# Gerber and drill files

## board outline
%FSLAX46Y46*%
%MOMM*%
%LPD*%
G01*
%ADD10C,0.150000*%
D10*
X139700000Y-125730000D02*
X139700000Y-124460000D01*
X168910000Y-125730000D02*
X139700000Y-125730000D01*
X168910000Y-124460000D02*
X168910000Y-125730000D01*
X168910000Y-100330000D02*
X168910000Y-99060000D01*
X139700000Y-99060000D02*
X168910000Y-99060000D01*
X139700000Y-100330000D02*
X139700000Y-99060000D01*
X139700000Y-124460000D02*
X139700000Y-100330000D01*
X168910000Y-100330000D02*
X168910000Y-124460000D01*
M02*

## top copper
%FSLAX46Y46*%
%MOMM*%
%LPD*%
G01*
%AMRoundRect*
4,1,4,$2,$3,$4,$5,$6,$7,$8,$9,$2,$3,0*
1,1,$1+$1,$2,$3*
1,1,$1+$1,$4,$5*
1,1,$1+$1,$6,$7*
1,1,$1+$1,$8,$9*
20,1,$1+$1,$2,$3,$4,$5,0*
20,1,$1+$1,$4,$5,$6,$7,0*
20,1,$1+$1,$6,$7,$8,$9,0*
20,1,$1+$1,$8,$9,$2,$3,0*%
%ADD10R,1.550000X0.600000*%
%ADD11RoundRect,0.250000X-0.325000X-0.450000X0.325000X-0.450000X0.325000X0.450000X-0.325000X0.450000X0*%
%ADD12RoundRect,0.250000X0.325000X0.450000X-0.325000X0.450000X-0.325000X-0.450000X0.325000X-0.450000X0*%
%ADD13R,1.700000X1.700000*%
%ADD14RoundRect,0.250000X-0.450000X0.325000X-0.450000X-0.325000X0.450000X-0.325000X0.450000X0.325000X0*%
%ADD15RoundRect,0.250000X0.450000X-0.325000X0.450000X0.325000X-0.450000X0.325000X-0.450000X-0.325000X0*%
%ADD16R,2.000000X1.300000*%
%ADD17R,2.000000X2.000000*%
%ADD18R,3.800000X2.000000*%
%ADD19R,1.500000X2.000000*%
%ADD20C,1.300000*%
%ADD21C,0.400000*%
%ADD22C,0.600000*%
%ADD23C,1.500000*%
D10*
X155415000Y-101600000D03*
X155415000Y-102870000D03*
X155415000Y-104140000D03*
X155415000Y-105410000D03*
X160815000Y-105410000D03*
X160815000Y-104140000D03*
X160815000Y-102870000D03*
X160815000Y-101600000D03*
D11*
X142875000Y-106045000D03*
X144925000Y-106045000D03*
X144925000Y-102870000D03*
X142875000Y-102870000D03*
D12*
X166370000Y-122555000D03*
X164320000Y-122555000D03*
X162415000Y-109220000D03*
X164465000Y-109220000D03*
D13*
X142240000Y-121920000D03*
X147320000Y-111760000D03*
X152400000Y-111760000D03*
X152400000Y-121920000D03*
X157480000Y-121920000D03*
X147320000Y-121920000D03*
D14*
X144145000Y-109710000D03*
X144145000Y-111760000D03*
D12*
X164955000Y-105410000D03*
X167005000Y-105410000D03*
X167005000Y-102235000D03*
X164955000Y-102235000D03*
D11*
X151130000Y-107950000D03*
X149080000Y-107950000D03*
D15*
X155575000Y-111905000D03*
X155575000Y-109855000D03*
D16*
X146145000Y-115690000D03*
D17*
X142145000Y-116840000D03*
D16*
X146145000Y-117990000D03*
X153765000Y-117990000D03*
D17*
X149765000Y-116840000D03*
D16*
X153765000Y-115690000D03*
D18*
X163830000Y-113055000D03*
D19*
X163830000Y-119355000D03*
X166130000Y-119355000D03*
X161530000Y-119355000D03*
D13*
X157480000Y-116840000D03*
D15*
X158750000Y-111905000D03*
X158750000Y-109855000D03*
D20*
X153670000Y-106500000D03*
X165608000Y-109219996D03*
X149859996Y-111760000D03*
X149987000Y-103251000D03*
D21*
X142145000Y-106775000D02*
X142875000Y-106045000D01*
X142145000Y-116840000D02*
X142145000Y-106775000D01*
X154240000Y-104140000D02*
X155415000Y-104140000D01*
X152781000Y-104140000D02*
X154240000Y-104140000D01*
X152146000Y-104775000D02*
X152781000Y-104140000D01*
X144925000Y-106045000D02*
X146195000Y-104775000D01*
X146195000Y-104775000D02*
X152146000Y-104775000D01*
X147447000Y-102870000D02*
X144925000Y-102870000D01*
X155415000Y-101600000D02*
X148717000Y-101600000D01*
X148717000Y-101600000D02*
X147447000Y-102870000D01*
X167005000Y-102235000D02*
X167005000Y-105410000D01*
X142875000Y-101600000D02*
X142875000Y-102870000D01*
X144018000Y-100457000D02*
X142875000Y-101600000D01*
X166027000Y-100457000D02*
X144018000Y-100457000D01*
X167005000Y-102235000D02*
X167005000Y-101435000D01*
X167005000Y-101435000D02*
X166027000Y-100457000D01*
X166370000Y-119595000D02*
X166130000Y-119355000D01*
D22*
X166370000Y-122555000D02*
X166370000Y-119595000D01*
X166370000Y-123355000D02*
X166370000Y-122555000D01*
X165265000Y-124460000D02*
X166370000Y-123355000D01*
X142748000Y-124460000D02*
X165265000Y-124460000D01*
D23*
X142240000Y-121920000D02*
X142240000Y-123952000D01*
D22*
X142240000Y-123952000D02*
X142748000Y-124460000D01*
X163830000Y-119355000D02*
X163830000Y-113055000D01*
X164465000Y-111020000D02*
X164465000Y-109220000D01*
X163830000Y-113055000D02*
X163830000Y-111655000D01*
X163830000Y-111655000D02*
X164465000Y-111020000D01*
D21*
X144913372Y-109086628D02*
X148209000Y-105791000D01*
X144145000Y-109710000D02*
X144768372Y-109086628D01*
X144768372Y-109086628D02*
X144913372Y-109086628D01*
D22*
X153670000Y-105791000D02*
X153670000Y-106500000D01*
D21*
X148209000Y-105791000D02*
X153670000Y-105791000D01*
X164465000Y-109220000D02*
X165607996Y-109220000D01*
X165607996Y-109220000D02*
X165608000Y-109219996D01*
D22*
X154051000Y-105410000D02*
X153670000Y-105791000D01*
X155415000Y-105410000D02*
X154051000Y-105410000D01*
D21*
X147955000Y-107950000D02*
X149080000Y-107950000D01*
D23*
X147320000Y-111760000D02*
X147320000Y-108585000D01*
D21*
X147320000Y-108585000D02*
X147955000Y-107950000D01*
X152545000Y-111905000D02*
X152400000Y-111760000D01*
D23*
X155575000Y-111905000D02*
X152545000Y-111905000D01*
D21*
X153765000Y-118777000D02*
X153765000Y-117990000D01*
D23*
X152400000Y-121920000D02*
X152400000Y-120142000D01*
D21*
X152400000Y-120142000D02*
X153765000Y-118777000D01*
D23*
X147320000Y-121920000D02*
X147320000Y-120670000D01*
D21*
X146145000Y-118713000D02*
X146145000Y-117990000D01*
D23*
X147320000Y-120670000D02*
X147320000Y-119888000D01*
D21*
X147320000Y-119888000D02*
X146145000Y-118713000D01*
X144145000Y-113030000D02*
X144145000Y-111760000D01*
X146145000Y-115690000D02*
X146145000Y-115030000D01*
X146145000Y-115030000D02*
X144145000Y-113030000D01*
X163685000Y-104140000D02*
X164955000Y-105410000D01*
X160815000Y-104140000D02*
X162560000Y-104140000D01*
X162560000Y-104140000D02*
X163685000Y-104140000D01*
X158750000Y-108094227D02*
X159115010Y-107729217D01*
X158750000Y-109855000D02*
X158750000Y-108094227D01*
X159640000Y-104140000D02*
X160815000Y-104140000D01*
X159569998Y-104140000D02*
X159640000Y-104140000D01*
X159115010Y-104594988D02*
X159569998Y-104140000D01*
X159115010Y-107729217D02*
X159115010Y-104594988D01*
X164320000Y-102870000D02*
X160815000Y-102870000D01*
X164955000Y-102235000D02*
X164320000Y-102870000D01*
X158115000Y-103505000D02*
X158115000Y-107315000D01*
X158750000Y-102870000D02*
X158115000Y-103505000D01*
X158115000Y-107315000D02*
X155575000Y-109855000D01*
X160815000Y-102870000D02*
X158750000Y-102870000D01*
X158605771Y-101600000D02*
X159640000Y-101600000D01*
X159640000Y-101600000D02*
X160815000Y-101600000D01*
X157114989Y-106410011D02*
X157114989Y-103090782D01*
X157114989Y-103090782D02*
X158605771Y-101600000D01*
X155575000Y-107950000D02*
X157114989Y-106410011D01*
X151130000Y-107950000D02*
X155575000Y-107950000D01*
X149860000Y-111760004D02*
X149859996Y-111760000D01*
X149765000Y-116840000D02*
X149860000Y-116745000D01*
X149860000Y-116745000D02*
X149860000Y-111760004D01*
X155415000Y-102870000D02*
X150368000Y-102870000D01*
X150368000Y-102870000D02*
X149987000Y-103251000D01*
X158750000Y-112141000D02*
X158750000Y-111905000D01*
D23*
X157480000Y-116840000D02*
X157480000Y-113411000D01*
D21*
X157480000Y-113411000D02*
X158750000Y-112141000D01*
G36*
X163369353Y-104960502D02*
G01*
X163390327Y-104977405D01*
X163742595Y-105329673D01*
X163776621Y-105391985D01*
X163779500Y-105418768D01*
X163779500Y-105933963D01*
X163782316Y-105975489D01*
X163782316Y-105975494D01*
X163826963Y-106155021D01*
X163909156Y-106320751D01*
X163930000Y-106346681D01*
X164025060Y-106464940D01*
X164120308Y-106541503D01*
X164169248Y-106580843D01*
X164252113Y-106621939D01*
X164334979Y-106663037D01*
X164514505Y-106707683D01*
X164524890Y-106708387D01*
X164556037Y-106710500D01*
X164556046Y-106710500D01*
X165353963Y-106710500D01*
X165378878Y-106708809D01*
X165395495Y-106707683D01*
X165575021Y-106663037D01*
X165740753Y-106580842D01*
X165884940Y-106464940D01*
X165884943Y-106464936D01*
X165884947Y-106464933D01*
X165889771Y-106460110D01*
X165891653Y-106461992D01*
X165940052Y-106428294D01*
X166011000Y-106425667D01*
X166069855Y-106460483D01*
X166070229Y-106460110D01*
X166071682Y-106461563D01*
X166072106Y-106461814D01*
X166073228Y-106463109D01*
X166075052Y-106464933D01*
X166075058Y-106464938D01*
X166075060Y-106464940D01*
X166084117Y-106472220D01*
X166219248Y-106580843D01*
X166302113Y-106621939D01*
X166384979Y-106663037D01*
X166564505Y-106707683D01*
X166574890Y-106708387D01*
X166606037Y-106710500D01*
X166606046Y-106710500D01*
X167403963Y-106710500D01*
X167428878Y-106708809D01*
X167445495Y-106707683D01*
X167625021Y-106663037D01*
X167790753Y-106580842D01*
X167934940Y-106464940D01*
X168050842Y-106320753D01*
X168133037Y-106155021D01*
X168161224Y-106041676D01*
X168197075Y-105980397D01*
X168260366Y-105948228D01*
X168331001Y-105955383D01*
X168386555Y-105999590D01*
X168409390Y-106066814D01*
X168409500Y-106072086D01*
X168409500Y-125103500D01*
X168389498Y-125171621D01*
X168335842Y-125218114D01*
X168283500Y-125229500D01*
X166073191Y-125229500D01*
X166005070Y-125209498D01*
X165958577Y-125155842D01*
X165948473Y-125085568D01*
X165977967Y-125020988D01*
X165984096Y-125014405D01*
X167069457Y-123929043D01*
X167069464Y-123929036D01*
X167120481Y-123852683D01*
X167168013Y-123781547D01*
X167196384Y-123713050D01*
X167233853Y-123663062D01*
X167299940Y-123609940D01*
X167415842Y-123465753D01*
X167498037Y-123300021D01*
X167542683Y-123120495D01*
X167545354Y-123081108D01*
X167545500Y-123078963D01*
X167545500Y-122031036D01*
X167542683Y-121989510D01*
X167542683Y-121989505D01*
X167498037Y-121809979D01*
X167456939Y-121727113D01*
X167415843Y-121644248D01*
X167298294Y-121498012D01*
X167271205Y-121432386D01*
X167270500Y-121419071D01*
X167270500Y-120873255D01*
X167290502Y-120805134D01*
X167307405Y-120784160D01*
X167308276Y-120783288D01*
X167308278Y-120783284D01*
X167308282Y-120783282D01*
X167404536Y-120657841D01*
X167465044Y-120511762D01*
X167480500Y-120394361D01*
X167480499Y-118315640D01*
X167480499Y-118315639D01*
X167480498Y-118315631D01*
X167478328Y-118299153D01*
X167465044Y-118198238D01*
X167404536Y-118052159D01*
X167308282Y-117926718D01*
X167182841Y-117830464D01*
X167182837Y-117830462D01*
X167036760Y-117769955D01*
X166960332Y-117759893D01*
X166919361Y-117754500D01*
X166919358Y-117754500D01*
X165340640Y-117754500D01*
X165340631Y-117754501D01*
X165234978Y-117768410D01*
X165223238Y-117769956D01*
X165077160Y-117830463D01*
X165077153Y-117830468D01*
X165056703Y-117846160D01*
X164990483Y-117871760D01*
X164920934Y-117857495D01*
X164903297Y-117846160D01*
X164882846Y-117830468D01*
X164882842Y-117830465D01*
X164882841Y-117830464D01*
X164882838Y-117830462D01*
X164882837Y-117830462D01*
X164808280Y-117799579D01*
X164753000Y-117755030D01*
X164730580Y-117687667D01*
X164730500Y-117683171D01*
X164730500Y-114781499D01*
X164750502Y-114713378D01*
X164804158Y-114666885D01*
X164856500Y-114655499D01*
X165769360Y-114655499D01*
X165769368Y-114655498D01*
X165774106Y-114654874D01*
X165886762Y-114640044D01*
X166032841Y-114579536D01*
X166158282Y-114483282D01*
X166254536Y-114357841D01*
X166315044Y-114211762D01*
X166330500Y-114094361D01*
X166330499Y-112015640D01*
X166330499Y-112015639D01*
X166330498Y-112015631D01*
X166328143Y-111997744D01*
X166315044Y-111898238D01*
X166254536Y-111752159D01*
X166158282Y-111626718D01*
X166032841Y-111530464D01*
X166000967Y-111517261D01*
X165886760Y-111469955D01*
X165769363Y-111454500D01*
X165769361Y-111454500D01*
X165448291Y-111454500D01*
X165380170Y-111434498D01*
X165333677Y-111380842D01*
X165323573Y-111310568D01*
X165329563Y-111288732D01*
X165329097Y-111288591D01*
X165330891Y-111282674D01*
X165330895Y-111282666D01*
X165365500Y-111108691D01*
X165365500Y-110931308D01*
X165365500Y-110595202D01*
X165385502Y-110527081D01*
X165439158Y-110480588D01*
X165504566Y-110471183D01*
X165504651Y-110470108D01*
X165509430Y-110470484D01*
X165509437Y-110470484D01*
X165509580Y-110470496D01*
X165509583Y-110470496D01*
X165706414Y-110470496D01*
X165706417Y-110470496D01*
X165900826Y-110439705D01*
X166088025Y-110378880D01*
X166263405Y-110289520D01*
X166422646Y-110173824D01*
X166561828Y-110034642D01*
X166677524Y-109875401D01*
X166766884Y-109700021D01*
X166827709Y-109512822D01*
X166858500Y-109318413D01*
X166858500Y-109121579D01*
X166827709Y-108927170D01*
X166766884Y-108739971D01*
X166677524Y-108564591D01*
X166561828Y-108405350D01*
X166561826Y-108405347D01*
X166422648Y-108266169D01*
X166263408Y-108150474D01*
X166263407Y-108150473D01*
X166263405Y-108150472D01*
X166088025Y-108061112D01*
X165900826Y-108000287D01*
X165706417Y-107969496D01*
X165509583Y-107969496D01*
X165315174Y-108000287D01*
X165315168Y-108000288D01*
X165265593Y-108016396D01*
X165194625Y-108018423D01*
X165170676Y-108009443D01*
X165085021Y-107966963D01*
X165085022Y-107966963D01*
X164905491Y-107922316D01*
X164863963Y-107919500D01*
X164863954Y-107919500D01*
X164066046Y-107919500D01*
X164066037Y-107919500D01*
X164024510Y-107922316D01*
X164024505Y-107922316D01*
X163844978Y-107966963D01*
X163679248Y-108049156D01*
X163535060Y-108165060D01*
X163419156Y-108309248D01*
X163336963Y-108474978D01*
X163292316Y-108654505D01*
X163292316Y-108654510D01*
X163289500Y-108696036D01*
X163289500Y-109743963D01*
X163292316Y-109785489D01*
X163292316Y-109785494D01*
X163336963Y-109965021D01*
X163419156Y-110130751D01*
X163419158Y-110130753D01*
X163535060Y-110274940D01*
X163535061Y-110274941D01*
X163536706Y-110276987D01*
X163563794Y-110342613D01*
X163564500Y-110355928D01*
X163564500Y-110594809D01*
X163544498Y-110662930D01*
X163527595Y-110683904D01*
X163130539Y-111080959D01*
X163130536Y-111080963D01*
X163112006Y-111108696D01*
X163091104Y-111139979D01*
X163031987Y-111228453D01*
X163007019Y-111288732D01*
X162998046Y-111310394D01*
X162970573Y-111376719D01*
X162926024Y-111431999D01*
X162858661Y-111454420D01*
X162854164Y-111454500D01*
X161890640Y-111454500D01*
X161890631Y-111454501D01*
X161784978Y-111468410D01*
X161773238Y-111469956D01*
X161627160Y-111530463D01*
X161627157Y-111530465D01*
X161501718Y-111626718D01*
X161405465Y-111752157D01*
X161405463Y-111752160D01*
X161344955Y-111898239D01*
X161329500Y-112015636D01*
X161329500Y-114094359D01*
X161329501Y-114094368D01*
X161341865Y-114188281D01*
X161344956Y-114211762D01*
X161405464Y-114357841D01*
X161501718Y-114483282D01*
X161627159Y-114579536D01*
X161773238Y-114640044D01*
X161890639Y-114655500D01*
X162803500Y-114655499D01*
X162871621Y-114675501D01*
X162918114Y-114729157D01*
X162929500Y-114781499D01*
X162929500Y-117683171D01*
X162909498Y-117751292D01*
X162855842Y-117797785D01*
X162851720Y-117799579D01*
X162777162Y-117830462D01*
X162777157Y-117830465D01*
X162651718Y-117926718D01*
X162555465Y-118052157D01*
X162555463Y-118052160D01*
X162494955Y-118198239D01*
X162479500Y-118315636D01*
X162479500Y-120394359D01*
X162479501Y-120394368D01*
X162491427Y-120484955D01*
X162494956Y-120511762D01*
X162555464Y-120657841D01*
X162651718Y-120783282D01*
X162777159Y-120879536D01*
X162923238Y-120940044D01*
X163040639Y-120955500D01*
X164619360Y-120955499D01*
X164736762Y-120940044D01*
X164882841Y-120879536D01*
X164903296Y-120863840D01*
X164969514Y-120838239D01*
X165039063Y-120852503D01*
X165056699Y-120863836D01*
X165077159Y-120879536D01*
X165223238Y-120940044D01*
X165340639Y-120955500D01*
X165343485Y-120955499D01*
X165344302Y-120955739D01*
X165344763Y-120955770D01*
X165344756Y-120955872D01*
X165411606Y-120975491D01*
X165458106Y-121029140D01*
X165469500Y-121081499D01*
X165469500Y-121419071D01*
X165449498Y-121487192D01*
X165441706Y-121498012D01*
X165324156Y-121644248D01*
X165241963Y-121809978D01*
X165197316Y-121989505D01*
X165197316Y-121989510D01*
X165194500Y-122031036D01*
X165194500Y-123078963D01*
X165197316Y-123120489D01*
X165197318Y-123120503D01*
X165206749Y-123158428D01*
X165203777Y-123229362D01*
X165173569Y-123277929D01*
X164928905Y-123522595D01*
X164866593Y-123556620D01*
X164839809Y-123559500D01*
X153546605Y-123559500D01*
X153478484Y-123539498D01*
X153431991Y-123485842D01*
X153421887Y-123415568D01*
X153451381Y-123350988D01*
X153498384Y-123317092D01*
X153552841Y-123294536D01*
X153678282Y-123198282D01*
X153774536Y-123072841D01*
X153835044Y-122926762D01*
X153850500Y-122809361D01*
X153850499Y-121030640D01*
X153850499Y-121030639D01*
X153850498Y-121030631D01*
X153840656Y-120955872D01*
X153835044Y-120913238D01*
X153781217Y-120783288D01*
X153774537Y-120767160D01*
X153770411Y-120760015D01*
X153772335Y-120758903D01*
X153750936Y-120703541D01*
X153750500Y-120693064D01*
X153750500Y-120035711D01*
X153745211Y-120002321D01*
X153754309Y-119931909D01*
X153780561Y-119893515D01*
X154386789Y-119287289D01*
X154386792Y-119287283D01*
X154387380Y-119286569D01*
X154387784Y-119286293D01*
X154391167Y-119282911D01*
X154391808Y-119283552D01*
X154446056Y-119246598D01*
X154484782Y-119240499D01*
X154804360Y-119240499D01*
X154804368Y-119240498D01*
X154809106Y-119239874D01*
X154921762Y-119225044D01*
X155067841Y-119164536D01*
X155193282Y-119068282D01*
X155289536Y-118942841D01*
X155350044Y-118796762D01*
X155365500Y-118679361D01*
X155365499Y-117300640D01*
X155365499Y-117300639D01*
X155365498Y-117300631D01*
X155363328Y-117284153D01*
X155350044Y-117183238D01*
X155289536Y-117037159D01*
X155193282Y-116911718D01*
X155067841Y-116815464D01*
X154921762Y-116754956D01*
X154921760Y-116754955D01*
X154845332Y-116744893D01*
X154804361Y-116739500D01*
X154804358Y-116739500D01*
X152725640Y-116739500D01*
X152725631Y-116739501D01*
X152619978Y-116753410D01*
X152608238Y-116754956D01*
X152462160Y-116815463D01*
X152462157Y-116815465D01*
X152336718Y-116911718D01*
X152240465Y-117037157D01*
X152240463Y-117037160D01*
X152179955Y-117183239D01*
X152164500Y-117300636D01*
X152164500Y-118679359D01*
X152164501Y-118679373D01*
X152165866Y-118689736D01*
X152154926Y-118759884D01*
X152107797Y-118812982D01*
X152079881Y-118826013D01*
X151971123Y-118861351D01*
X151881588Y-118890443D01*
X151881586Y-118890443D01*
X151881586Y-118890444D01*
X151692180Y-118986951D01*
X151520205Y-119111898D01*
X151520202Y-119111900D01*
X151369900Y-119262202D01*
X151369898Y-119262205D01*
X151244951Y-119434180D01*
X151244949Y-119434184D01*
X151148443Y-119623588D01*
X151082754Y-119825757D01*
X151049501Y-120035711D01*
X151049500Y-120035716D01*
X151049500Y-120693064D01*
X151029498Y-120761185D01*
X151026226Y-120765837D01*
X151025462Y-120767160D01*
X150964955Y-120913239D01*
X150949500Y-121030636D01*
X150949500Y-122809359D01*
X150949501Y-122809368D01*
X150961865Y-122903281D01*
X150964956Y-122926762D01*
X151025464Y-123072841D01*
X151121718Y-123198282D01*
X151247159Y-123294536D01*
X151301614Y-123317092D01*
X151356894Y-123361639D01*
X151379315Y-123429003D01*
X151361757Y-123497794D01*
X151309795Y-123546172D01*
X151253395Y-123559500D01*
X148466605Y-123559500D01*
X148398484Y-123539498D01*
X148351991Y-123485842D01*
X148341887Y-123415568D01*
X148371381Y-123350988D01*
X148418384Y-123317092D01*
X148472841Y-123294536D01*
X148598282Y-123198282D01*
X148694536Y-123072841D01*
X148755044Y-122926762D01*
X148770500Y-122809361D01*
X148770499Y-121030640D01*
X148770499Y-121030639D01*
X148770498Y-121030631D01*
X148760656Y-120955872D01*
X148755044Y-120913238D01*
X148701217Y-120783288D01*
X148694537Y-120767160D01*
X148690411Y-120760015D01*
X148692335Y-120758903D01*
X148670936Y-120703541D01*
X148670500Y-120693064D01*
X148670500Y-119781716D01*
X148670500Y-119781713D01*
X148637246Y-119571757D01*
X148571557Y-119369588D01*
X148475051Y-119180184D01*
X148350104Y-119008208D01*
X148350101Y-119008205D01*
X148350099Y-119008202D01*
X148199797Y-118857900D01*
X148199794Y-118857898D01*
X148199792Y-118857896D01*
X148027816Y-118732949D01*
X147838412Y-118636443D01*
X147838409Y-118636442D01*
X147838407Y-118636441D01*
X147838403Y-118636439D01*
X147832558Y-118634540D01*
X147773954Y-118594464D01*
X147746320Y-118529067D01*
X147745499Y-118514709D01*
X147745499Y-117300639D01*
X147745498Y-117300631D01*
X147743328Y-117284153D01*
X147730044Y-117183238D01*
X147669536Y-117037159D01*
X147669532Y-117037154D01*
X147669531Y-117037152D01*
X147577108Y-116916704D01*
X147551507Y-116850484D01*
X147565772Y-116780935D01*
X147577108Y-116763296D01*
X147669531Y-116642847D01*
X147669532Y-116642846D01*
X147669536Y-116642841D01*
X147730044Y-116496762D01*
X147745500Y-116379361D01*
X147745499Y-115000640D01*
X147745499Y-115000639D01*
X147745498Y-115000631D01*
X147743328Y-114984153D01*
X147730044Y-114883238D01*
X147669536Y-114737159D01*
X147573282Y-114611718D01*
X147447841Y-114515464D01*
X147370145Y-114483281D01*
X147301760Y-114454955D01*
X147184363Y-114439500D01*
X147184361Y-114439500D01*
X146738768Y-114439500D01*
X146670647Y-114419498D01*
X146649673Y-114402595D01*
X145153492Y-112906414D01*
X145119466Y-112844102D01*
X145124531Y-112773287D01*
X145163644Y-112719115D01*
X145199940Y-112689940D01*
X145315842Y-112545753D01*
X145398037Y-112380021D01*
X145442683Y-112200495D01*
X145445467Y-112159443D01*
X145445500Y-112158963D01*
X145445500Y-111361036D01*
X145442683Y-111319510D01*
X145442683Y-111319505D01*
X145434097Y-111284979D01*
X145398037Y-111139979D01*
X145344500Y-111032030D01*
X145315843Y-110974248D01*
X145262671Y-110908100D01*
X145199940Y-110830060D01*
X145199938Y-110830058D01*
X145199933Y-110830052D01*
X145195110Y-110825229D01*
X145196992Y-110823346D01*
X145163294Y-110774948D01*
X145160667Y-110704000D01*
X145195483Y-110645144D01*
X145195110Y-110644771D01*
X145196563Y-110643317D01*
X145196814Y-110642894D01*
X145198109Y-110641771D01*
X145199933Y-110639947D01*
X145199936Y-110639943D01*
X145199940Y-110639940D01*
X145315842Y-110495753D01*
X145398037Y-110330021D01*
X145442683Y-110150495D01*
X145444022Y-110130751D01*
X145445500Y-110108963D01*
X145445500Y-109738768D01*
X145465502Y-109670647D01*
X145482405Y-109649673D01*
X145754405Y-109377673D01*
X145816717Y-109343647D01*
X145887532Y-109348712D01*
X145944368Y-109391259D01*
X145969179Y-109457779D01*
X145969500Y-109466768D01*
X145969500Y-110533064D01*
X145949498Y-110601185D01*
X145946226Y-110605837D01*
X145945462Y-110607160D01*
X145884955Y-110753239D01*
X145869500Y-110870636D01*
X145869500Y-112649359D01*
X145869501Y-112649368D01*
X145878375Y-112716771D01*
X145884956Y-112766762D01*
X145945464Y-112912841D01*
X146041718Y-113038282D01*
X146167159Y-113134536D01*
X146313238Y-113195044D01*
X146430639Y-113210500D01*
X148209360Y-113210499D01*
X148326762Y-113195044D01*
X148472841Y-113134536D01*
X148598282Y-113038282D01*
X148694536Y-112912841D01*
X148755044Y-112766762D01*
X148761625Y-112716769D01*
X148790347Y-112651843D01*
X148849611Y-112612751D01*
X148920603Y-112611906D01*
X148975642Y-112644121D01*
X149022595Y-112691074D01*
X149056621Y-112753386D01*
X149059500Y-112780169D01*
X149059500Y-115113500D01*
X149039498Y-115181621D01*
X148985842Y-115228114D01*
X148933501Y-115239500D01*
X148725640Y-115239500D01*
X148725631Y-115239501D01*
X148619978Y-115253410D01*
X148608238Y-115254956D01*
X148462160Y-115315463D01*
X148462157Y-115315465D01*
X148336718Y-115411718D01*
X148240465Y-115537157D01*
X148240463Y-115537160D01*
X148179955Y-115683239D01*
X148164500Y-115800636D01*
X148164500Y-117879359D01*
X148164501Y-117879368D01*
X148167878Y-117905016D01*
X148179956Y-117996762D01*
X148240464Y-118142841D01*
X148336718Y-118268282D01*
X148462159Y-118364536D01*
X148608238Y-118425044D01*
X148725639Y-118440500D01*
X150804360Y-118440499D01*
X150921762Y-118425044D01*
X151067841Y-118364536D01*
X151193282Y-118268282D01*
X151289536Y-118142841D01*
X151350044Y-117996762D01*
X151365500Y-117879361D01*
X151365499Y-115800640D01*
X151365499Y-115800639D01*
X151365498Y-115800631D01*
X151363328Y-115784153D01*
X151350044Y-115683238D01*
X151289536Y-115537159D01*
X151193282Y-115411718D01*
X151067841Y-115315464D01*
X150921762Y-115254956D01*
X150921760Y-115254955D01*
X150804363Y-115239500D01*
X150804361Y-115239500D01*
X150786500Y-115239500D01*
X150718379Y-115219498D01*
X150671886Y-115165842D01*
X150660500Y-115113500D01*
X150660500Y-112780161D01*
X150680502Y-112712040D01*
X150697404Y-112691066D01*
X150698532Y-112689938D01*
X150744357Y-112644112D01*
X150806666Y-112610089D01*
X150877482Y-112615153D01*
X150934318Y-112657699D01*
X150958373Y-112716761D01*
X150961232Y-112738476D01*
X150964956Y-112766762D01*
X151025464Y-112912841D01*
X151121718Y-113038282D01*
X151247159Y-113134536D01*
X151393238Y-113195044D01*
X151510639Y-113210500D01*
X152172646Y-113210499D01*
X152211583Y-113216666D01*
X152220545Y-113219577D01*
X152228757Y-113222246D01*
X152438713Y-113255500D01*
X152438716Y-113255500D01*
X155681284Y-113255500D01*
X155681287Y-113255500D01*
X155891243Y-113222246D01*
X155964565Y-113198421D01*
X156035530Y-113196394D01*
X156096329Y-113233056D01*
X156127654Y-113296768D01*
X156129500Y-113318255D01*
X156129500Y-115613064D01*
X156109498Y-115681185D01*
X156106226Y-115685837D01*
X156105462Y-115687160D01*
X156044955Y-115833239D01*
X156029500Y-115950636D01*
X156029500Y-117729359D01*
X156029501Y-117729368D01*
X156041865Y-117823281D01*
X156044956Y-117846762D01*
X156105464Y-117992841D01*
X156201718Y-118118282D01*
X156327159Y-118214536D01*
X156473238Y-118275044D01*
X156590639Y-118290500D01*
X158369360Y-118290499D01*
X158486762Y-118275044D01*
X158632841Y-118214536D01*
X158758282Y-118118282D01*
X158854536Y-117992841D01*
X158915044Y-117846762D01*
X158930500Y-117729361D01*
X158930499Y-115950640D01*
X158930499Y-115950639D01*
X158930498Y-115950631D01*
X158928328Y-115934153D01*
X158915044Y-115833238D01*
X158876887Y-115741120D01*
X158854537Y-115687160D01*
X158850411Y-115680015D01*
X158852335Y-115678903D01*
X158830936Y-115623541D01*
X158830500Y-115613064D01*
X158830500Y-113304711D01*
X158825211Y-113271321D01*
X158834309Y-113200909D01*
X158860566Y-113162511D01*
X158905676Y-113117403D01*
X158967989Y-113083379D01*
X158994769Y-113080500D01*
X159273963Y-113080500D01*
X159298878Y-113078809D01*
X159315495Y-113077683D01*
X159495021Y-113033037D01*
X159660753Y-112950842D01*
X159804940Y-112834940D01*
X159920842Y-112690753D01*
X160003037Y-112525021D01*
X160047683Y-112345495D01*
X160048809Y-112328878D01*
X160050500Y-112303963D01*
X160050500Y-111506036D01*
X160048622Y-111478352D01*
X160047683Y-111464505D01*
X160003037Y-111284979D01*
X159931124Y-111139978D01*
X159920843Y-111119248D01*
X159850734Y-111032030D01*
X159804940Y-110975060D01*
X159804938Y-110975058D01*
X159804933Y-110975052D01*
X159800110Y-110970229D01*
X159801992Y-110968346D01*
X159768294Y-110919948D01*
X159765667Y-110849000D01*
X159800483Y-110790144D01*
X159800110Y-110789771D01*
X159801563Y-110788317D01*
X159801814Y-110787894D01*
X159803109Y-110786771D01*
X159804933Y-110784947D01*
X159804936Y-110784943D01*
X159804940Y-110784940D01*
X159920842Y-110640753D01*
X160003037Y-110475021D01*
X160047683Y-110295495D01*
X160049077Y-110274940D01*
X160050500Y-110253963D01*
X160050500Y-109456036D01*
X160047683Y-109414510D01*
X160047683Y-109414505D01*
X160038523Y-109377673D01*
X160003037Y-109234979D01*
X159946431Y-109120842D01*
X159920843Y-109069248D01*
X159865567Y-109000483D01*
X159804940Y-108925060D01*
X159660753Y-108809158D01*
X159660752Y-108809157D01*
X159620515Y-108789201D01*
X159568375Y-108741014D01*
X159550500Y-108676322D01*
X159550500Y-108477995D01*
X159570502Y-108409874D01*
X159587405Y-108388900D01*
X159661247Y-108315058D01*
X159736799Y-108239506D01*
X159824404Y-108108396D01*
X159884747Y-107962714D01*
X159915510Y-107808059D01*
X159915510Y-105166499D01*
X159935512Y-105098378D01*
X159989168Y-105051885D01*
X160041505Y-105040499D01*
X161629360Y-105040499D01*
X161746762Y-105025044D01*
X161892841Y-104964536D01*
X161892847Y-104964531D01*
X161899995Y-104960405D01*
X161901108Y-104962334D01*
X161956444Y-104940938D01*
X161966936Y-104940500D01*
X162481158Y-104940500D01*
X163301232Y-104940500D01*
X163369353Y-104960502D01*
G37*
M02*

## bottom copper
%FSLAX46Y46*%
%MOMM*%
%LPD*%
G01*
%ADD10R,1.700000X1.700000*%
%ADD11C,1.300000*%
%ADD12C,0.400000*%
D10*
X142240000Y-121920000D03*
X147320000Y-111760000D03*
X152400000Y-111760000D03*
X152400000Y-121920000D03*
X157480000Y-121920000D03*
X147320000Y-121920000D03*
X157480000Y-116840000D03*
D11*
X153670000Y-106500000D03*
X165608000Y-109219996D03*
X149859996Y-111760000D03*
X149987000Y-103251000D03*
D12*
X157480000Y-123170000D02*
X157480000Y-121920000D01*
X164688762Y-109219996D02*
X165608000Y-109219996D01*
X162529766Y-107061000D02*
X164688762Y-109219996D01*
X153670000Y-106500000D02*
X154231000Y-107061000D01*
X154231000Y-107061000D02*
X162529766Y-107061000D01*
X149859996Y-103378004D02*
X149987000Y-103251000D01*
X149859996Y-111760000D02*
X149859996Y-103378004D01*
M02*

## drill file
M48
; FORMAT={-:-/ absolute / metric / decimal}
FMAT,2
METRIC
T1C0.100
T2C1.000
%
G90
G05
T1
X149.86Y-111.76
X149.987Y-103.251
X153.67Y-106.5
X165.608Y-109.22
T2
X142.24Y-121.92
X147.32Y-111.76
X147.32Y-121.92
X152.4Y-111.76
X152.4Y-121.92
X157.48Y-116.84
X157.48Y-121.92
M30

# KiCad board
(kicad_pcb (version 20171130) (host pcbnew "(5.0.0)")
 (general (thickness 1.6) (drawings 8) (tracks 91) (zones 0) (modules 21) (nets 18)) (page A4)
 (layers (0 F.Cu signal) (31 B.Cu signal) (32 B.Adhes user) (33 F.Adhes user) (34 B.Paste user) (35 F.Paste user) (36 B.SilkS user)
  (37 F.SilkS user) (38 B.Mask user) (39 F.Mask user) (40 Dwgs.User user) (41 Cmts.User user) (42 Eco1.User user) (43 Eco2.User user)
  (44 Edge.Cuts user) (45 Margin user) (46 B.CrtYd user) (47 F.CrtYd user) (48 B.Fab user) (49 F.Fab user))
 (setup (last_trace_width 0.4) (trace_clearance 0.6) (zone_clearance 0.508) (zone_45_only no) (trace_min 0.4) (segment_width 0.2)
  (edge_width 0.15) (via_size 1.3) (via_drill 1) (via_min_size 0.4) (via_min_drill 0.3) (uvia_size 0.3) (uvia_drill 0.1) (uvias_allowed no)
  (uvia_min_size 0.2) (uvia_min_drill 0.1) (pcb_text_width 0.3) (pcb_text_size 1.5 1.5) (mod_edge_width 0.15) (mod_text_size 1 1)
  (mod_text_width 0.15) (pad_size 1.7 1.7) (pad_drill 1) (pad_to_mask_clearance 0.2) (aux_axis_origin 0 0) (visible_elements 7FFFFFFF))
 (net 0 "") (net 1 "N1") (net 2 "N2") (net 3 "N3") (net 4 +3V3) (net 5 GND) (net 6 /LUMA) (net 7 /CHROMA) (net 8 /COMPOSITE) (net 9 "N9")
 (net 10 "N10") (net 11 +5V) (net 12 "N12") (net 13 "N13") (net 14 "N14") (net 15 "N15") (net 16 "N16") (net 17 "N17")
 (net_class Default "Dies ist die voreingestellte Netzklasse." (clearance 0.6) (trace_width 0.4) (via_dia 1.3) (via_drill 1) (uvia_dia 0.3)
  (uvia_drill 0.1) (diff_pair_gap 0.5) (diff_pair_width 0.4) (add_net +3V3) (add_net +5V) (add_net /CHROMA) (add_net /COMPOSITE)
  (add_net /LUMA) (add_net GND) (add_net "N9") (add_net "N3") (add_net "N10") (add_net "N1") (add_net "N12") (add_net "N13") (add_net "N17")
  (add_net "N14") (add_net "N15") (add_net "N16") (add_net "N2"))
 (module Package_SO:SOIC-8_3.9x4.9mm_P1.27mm (layer F.Cu) (at 158.115 103.505)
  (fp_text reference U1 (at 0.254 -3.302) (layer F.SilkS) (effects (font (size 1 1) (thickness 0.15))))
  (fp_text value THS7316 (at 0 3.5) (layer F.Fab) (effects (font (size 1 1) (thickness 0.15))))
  (pad 1 smd rect (at -2.7 -1.905) (size 1.55 0.6) (layers F.Cu F.Paste F.Mask) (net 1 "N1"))
  (pad 2 smd rect (at -2.7 -0.635) (size 1.55 0.6) (layers F.Cu F.Paste F.Mask) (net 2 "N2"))
  (pad 3 smd rect (at -2.7 0.635) (size 1.55 0.6) (layers F.Cu F.Paste F.Mask) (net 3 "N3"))
  (pad 4 smd rect (at -2.7 1.905) (size 1.55 0.6) (layers F.Cu F.Paste F.Mask) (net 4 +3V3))
  (pad 5 smd rect (at 2.7 1.905) (size 1.55 0.6) (layers F.Cu F.Paste F.Mask) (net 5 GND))
  (pad 6 smd rect (at 2.7 0.635) (size 1.55 0.6) (layers F.Cu F.Paste F.Mask) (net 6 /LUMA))
  (pad 7 smd rect (at 2.7 -0.635) (size 1.55 0.6) (layers F.Cu F.Paste F.Mask) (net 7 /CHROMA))
  (pad 8 smd rect (at 2.7 -1.905) (size 1.55 0.6) (layers F.Cu F.Paste F.Mask) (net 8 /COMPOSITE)))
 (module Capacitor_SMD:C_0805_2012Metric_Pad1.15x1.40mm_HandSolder (layer F.Cu) (at 143.9 106.045)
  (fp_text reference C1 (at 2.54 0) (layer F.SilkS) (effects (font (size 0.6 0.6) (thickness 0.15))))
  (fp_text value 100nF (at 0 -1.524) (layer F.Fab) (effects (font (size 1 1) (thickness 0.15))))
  (pad 1 smd roundrect (at -1.025 0) (size 1.15 1.4) (layers F.Cu F.Paste F.Mask) (roundrect_rratio 0.217391) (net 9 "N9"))
  (pad 2 smd roundrect (at 1.025 0) (size 1.15 1.4) (layers F.Cu F.Paste F.Mask) (roundrect_rratio 0.217391) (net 3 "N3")))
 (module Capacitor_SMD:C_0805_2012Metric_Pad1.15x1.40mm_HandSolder (layer F.Cu) (at 143.9 102.87)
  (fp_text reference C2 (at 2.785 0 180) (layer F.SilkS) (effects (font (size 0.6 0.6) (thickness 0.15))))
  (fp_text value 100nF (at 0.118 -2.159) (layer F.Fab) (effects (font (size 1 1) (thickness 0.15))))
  (pad 2 smd roundrect (at 1.025 0) (size 1.15 1.4) (layers F.Cu F.Paste F.Mask) (roundrect_rratio 0.217391) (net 1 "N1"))
  (pad 1 smd roundrect (at -1.025 0) (size 1.15 1.4) (layers F.Cu F.Paste F.Mask) (roundrect_rratio 0.217391) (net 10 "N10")))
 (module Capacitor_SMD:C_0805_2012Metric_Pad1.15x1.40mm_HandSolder (layer F.Cu) (at 165.345 122.555 180)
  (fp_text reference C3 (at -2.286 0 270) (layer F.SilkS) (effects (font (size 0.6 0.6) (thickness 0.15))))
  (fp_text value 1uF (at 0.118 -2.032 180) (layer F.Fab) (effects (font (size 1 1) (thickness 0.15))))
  (pad 1 smd roundrect (at -1.025 0 180) (size 1.15 1.4) (layers F.Cu F.Paste F.Mask) (roundrect_rratio 0.217391) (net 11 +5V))
  (pad 2 smd roundrect (at 1.025 0 180) (size 1.15 1.4) (layers F.Cu F.Paste F.Mask) (roundrect_rratio 0.217391) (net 5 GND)))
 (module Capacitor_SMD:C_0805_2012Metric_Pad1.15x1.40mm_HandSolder (layer F.Cu) (at 163.44 109.22 180)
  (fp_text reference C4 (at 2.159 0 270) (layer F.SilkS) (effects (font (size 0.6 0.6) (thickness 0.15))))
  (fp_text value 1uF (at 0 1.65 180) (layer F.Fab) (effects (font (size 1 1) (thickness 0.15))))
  (pad 2 smd roundrect (at 1.025 0 180) (size 1.15 1.4) (layers F.Cu F.Paste F.Mask) (roundrect_rratio 0.217391) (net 5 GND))
  (pad 1 smd roundrect (at -1.025 0 180) (size 1.15 1.4) (layers F.Cu F.Paste F.Mask) (roundrect_rratio 0.217391) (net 4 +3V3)))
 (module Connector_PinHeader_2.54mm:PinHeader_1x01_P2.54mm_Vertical (layer B.Cu) (at 142.24 121.92)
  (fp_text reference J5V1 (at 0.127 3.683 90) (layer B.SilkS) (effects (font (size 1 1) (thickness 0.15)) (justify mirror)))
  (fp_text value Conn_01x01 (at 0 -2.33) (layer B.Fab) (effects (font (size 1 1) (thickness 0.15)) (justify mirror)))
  (pad 1 thru_hole rect (at 0 0) (size 1.7 1.7) (drill 1) (layers *.Cu *.Mask) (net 11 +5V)))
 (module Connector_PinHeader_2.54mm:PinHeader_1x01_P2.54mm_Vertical (layer B.Cu) (at 147.32 111.76)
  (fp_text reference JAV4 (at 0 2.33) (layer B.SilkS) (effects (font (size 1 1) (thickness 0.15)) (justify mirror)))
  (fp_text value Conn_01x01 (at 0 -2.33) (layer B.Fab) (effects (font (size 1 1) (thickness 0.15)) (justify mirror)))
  (pad 1 thru_hole rect (at 0 0) (size 1.7 1.7) (drill 1) (layers *.Cu *.Mask) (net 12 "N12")))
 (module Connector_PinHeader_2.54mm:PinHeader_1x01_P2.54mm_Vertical (layer B.Cu) (at 152.4 111.76)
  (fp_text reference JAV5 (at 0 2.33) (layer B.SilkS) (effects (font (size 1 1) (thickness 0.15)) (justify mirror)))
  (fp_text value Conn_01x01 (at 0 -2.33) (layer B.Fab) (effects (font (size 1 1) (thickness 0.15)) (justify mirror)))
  (pad 1 thru_hole rect (at 0 0) (size 1.7 1.7) (drill 1) (layers *.Cu *.Mask) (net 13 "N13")))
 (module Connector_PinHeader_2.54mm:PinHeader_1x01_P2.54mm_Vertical (layer B.Cu) (at 152.4 121.92)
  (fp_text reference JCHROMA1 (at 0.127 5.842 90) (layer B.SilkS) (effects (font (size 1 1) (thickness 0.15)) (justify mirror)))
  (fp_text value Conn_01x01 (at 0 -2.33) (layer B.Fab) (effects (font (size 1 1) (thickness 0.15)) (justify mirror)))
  (pad 1 thru_hole rect (at 0 0) (size 1.7 1.7) (drill 1) (layers *.Cu *.Mask) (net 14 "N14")))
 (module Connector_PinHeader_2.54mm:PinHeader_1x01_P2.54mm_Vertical (layer B.Cu) (at 157.48 121.92)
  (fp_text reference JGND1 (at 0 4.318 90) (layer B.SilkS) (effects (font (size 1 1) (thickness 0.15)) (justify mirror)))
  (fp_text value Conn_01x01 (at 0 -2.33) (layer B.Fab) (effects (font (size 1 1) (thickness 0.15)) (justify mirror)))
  (pad 1 thru_hole rect (at 0 0) (size 1.7 1.7) (drill 1) (layers *.Cu *.Mask) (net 5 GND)))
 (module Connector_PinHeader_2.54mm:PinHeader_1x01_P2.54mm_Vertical (layer B.Cu) (at 147.32 121.92)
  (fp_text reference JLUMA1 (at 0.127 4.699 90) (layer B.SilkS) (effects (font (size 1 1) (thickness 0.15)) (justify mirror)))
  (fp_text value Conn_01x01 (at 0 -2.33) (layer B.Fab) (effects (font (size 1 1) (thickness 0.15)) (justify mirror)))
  (pad 1 thru_hole rect (at 0 0) (size 1.7 1.7) (drill 1) (layers *.Cu *.Mask) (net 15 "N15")))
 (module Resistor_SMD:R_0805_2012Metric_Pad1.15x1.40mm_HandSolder (layer F.Cu) (at 144.145 110.735 270)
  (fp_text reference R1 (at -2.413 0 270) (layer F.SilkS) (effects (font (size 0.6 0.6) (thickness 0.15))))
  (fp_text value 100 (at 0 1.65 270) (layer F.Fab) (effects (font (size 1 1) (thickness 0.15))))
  (pad 1 smd roundrect (at -1.025 0 270) (size 1.15 1.4) (layers F.Cu F.Paste F.Mask) (roundrect_rratio 0.217391) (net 4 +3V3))
  (pad 2 smd roundrect (at 1.025 0 270) (size 1.15 1.4) (layers F.Cu F.Paste F.Mask) (roundrect_rratio 0.217391) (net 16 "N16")))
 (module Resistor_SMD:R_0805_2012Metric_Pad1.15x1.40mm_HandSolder (layer F.Cu) (at 165.98 105.41 180)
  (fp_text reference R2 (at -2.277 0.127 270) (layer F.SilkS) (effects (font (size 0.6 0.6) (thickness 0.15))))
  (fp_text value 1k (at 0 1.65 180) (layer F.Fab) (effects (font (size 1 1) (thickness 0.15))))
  (pad 2 smd roundrect (at 1.025 0 180) (size 1.15 1.4) (layers F.Cu F.Paste F.Mask) (roundrect_rratio 0.217391) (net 6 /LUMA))
  (pad 1 smd roundrect (at -1.025 0 180) (size 1.15 1.4) (layers F.Cu F.Paste F.Mask) (roundrect_rratio 0.217391) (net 10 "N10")))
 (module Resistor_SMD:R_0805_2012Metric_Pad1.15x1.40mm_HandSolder (layer F.Cu) (at 165.98 102.235 180)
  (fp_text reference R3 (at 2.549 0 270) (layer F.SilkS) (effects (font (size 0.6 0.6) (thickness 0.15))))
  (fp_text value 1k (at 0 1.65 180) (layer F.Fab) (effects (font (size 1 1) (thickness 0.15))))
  (pad 1 smd roundrect (at -1.025 0 180) (size 1.15 1.4) (layers F.Cu F.Paste F.Mask) (roundrect_rratio 0.217391) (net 10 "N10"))
  (pad 2 smd roundrect (at 1.025 0 180) (size 1.15 1.4) (layers F.Cu F.Paste F.Mask) (roundrect_rratio 0.217391) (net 7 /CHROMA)))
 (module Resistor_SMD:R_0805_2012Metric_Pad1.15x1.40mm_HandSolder (layer F.Cu) (at 150.105 107.95)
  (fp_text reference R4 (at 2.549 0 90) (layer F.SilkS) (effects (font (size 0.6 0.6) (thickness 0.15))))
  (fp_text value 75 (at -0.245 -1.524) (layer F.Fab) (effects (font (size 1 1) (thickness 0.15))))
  (pad 2 smd roundrect (at 1.025 0) (size 1.15 1.4) (layers F.Cu F.Paste F.Mask) (roundrect_rratio 0.217391) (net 8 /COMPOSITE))
  (pad 1 smd roundrect (at -1.025 0) (size 1.15 1.4) (layers F.Cu F.Paste F.Mask) (roundrect_rratio 0.217391) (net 12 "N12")))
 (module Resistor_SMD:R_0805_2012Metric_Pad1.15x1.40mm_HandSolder (layer F.Cu) (at 155.575 110.88 90)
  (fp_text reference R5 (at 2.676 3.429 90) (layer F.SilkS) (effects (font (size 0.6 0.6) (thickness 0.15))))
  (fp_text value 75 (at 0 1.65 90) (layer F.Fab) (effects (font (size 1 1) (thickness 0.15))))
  (pad 1 smd roundrect (at -1.025 0 90) (size 1.15 1.4) (layers F.Cu F.Paste F.Mask) (roundrect_rratio 0.217391) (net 13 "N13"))
  (pad 2 smd roundrect (at 1.025 0 90) (size 1.15 1.4) (layers F.Cu F.Paste F.Mask) (roundrect_rratio 0.217391) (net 7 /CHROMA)))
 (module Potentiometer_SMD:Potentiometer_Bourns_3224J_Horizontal (layer F.Cu) (at 144.145 116.84)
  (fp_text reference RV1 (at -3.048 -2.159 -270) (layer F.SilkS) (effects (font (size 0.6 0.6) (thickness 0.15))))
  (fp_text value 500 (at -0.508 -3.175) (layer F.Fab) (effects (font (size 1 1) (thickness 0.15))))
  (pad 1 smd rect (at 2 -1.15) (size 2 1.3) (layers F.Cu F.Paste F.Mask) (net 16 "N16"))
  (pad 2 smd rect (at -2 0) (size 2 2) (layers F.Cu F.Paste F.Mask) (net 9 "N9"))
  (pad 3 smd rect (at 2 1.15) (size 2 1.3) (layers F.Cu F.Paste F.Mask) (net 15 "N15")))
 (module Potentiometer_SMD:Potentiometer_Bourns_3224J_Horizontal (layer F.Cu) (at 151.765 116.84)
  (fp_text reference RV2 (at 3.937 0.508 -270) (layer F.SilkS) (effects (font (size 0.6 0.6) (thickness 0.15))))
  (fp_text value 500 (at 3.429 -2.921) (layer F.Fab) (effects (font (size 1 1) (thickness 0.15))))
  (pad 3 smd rect (at 2 1.15) (size 2 1.3) (layers F.Cu F.Paste F.Mask) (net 14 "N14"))
  (pad 2 smd rect (at -2 0) (size 2 2) (layers F.Cu F.Paste F.Mask) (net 2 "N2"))
  (pad 1 smd rect (at 2 -1.15) (size 2 1.3) (layers F.Cu F.Paste F.Mask) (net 5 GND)))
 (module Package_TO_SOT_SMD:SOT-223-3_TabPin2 (layer F.Cu) (at 163.83 116.205 90)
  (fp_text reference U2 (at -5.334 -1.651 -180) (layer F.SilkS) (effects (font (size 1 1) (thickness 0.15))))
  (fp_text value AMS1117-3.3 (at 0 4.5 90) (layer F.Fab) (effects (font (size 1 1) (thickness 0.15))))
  (pad 2 smd rect (at 3.15 0 90) (size 2 3.8) (layers F.Cu F.Paste F.Mask) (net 4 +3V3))
  (pad 2 smd rect (at -3.15 0 90) (size 2 1.5) (layers F.Cu F.Paste F.Mask) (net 4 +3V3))
  (pad 3 smd rect (at -3.15 2.3 90) (size 2 1.5) (layers F.Cu F.Paste F.Mask) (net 11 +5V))
  (pad 1 smd rect (at -3.15 -2.3 90) (size 2 1.5) (layers F.Cu F.Paste F.Mask) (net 5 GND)))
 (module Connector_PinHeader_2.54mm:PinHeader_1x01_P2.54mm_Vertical (layer B.Cu) (at 157.48 116.84)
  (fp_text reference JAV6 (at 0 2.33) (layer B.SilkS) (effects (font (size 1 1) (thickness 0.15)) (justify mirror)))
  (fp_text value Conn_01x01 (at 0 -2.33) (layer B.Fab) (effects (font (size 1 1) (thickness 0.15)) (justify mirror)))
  (pad 1 thru_hole rect (at 0 0) (size 1.7 1.7) (drill 1) (layers *.Cu *.Mask) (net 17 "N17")))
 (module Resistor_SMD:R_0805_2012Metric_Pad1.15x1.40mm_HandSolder (layer F.Cu) (at 158.75 110.88 90)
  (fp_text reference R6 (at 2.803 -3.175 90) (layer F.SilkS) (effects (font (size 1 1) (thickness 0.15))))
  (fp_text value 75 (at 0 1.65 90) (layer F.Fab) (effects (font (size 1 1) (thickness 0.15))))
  (pad 1 smd roundrect (at -1.025 0 90) (size 1.15 1.4) (layers F.Cu F.Paste F.Mask) (roundrect_rratio 0.217391) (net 17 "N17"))
  (pad 2 smd roundrect (at 1.025 0 90) (size 1.15 1.4) (layers F.Cu F.Paste F.Mask) (roundrect_rratio 0.217391) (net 6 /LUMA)))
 (gr_line (start 139.7 125.73) (end 139.7 124.46) (layer Edge.Cuts) (width 0.15))
 (gr_line (start 168.91 125.73) (end 139.7 125.73) (layer Edge.Cuts) (width 0.15))
 (gr_line (start 168.91 124.46) (end 168.91 125.73) (layer Edge.Cuts) (width 0.15))
 (gr_line (start 168.91 100.33) (end 168.91 99.06) (layer Edge.Cuts) (width 0.15))
 (gr_line (start 139.7 99.06) (end 168.91 99.06) (layer Edge.Cuts) (width 0.15))
 (gr_line (start 139.7 100.33) (end 139.7 99.06) (layer Edge.Cuts) (width 0.15))
 (gr_line (start 139.7 124.46) (end 139.7 100.33) (layer Edge.Cuts) (width 0.15))
 (gr_line (start 168.91 100.33) (end 168.91 124.46) (layer Edge.Cuts) (width 0.15))
 (segment (start 142.145 106.775) (end 142.875 106.045) (width 0.4) (layer F.Cu) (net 9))
 (segment (start 142.145 116.84) (end 142.145 106.775) (width 0.4) (layer F.Cu) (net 9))
 (segment (start 154.24 104.14) (end 155.415 104.14) (width 0.4) (layer F.Cu) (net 3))
 (segment (start 152.781 104.14) (end 154.24 104.14) (width 0.4) (layer F.Cu) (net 3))
 (segment (start 152.146 104.775) (end 152.781 104.14) (width 0.4) (layer F.Cu) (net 3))
 (segment (start 144.925 106.045) (end 146.195 104.775) (width 0.4) (layer F.Cu) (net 3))
 (segment (start 146.195 104.775) (end 152.146 104.775) (width 0.4) (layer F.Cu) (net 3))
 (segment (start 147.447 102.87) (end 144.925 102.87) (width 0.4) (layer F.Cu) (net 1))
 (segment (start 155.415 101.6) (end 148.717 101.6) (width 0.4) (layer F.Cu) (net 1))
 (segment (start 148.717 101.6) (end 147.447 102.87) (width 0.4) (layer F.Cu) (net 1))
 (segment (start 167.005 102.235) (end 167.005 105.41) (width 0.4) (layer F.Cu) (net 10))
 (segment (start 142.875 101.6) (end 142.875 102.87) (width 0.4) (layer F.Cu) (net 10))
 (segment (start 144.018 100.457) (end 142.875 101.6) (width 0.4) (layer F.Cu) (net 10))
 (segment (start 166.027 100.457) (end 144.018 100.457) (width 0.4) (layer F.Cu) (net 10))
 (segment (start 167.005 102.235) (end 167.005 101.435) (width 0.4) (layer F.Cu) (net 10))
 (segment (start 167.005 101.435) (end 166.027 100.457) (width 0.4) (layer F.Cu) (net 10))
 (segment (start 166.37 119.595) (end 166.13 119.355) (width 0.4) (layer F.Cu) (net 11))
 (segment (start 166.37 122.555) (end 166.37 119.595) (width 0.6) (layer F.Cu) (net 11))
 (segment (start 166.37 123.355) (end 166.37 122.555) (width 0.6) (layer F.Cu) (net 11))
 (segment (start 165.265 124.46) (end 166.37 123.355) (width 0.6) (layer F.Cu) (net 11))
 (segment (start 142.748 124.46) (end 165.265 124.46) (width 0.6) (layer F.Cu) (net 11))
 (segment (start 142.24 121.92) (end 142.24 123.952) (width 1.5) (layer F.Cu) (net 11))
 (segment (start 142.24 123.952) (end 142.748 124.46) (width 0.6) (layer F.Cu) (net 11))
 (segment (start 157.48 123.17) (end 157.48 121.92) (width 0.4) (layer B.Cu) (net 5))
 (segment (start 163.83 119.355) (end 163.83 113.055) (width 0.6) (layer F.Cu) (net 4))
 (segment (start 164.465 111.02) (end 164.465 109.22) (width 0.6) (layer F.Cu) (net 4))
 (segment (start 163.83 113.055) (end 163.83 111.655) (width 0.6) (layer F.Cu) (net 4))
 (segment (start 163.83 111.655) (end 164.465 111.02) (width 0.6) (layer F.Cu) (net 4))
 (segment (start 144.913372 109.086628) (end 148.209 105.791) (width 0.4) (layer F.Cu) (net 4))
 (segment (start 144.145 109.71) (end 144.768372 109.086628) (width 0.4) (layer F.Cu) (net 4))
 (segment (start 144.768372 109.086628) (end 144.913372 109.086628) (width 0.4) (layer F.Cu) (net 4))
 (via (at 153.67 106.5) (size 1.3) (drill 0.1) (layers F.Cu B.Cu) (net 4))
 (segment (start 153.67 105.791) (end 153.67 106.5) (width 0.6) (layer F.Cu) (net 4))
 (segment (start 148.209 105.791) (end 153.67 105.791) (width 0.4) (layer F.Cu) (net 4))
 (via (at 165.608 109.219996) (size 1.3) (drill 0.1) (layers F.Cu B.Cu) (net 4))
 (segment (start 164.465 109.22) (end 165.607996 109.22) (width 0.4) (layer F.Cu) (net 4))
 (segment (start 165.607996 109.22) (end 165.608 109.219996) (width 0.4) (layer F.Cu) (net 4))
 (segment (start 164.688762 109.219996) (end 165.608 109.219996) (width 0.4) (layer B.Cu) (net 4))
 (segment (start 162.529766 107.061) (end 164.688762 109.219996) (width 0.4) (layer B.Cu) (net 4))
 (segment (start 153.67 106.5) (end 154.231 107.061) (width 0.4) (layer B.Cu) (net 4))
 (segment (start 154.231 107.061) (end 162.529766 107.061) (width 0.4) (layer B.Cu) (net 4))
 (segment (start 154.051 105.41) (end 153.67 105.791) (width 0.6) (layer F.Cu) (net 4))
 (segment (start 155.415 105.41) (end 154.051 105.41) (width 0.6) (layer F.Cu) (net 4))
 (segment (start 147.955 107.95) (end 149.08 107.95) (width 0.4) (layer F.Cu) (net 12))
 (segment (start 147.32 111.76) (end 147.32 108.585) (width 1.5) (layer F.Cu) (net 12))
 (segment (start 147.32 108.585) (end 147.955 107.95) (width 0.4) (layer F.Cu) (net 12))
 (segment (start 152.545 111.905) (end 152.4 111.76) (width 0.4) (layer F.Cu) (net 13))
 (segment (start 155.575 111.905) (end 152.545 111.905) (width 1.5) (layer F.Cu) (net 13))
 (segment (start 153.765 118.777) (end 153.765 117.99) (width 0.4) (layer F.Cu) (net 14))
 (segment (start 152.4 121.92) (end 152.4 120.142) (width 1.5) (layer F.Cu) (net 14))
 (segment (start 152.4 120.142) (end 153.765 118.777) (width 0.4) (layer F.Cu) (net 14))
 (segment (start 147.32 121.92) (end 147.32 120.67) (width 1.5) (layer F.Cu) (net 15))
 (segment (start 146.145 118.713) (end 146.145 117.99) (width 0.4) (layer F.Cu) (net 15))
 (segment (start 147.32 120.67) (end 147.32 119.888) (width 1.5) (layer F.Cu) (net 15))
 (segment (start 147.32 119.888) (end 146.145 118.713) (width 0.4) (layer F.Cu) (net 15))
 (segment (start 144.145 113.03) (end 144.145 111.76) (width 0.4) (layer F.Cu) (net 16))
 (segment (start 146.145 115.69) (end 146.145 115.03) (width 0.4) (layer F.Cu) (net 16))
 (segment (start 146.145 115.03) (end 144.145 113.03) (width 0.4) (layer F.Cu) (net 16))
 (segment (start 163.685 104.14) (end 164.955 105.41) (width 0.4) (layer F.Cu) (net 6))
 (segment (start 160.815 104.14) (end 162.56 104.14) (width 0.4) (layer F.Cu) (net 6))
 (segment (start 162.56 104.14) (end 163.685 104.14) (width 0.4) (layer F.Cu) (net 6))
 (segment (start 158.75 108.094227) (end 159.11501 107.729217) (width 0.4) (layer F.Cu) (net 6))
 (segment (start 158.75 109.855) (end 158.75 108.094227) (width 0.4) (layer F.Cu) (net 6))
 (segment (start 159.64 104.14) (end 160.815 104.14) (width 0.4) (layer F.Cu) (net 6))
 (segment (start 159.569998 104.14) (end 159.64 104.14) (width 0.4) (layer F.Cu) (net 6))
 (segment (start 159.11501 104.594988) (end 159.569998 104.14) (width 0.4) (layer F.Cu) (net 6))
 (segment (start 159.11501 107.729217) (end 159.11501 104.594988) (width 0.4) (layer F.Cu) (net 6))
 (segment (start 164.32 102.87) (end 160.815 102.87) (width 0.4) (layer F.Cu) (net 7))
 (segment (start 164.955 102.235) (end 164.32 102.87) (width 0.4) (layer F.Cu) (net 7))
 (segment (start 158.115 103.505) (end 158.115 107.315) (width 0.4) (layer F.Cu) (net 7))
 (segment (start 158.75 102.87) (end 158.115 103.505) (width 0.4) (layer F.Cu) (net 7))
 (segment (start 158.115 107.315) (end 155.575 109.855) (width 0.4) (layer F.Cu) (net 7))
 (segment (start 160.815 102.87) (end 158.75 102.87) (width 0.4) (layer F.Cu) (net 7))
 (segment (start 158.605771 101.6) (end 159.64 101.6) (width 0.4) (layer F.Cu) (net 8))
 (segment (start 159.64 101.6) (end 160.815 101.6) (width 0.4) (layer F.Cu) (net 8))
 (segment (start 157.114989 106.410011) (end 157.114989 103.090782) (width 0.4) (layer F.Cu) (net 8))
 (segment (start 157.114989 103.090782) (end 158.605771 101.6) (width 0.4) (layer F.Cu) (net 8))
 (segment (start 155.575 107.95) (end 157.114989 106.410011) (width 0.4) (layer F.Cu) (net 8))
 (segment (start 151.13 107.95) (end 155.575 107.95) (width 0.4) (layer F.Cu) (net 8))
 (via (at 149.859996 111.76) (size 1.3) (drill 0.1) (layers F.Cu B.Cu) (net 2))
 (segment (start 149.86 111.760004) (end 149.859996 111.76) (width 0.4) (layer F.Cu) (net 2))
 (segment (start 149.765 116.84) (end 149.86 116.745) (width 0.4) (layer F.Cu) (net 2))
 (segment (start 149.86 116.745) (end 149.86 111.760004) (width 0.4) (layer F.Cu) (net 2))
 (via (at 149.987 103.251) (size 1.3) (drill 0.1) (layers F.Cu B.Cu) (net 2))
 (segment (start 155.415 102.87) (end 150.368 102.87) (width 0.4) (layer F.Cu) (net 2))
 (segment (start 150.368 102.87) (end 149.987 103.251) (width 0.4) (layer F.Cu) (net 2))
 (segment (start 149.859996 103.378004) (end 149.987 103.251) (width 0.4) (layer B.Cu) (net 2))
 (segment (start 149.859996 111.76) (end 149.859996 103.378004) (width 0.4) (layer B.Cu) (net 2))
 (segment (start 158.75 112.141) (end 158.75 111.905) (width 0.4) (layer F.Cu) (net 17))
 (segment (start 157.48 116.84) (end 157.48 113.411) (width 1.5) (layer F.Cu) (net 17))
 (segment (start 157.48 113.411) (end 158.75 112.141) (width 0.4) (layer F.Cu) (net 17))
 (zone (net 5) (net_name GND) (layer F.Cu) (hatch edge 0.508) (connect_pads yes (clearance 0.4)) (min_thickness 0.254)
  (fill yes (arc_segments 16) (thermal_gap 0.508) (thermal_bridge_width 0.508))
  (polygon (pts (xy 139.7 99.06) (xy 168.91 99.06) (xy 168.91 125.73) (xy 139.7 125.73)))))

